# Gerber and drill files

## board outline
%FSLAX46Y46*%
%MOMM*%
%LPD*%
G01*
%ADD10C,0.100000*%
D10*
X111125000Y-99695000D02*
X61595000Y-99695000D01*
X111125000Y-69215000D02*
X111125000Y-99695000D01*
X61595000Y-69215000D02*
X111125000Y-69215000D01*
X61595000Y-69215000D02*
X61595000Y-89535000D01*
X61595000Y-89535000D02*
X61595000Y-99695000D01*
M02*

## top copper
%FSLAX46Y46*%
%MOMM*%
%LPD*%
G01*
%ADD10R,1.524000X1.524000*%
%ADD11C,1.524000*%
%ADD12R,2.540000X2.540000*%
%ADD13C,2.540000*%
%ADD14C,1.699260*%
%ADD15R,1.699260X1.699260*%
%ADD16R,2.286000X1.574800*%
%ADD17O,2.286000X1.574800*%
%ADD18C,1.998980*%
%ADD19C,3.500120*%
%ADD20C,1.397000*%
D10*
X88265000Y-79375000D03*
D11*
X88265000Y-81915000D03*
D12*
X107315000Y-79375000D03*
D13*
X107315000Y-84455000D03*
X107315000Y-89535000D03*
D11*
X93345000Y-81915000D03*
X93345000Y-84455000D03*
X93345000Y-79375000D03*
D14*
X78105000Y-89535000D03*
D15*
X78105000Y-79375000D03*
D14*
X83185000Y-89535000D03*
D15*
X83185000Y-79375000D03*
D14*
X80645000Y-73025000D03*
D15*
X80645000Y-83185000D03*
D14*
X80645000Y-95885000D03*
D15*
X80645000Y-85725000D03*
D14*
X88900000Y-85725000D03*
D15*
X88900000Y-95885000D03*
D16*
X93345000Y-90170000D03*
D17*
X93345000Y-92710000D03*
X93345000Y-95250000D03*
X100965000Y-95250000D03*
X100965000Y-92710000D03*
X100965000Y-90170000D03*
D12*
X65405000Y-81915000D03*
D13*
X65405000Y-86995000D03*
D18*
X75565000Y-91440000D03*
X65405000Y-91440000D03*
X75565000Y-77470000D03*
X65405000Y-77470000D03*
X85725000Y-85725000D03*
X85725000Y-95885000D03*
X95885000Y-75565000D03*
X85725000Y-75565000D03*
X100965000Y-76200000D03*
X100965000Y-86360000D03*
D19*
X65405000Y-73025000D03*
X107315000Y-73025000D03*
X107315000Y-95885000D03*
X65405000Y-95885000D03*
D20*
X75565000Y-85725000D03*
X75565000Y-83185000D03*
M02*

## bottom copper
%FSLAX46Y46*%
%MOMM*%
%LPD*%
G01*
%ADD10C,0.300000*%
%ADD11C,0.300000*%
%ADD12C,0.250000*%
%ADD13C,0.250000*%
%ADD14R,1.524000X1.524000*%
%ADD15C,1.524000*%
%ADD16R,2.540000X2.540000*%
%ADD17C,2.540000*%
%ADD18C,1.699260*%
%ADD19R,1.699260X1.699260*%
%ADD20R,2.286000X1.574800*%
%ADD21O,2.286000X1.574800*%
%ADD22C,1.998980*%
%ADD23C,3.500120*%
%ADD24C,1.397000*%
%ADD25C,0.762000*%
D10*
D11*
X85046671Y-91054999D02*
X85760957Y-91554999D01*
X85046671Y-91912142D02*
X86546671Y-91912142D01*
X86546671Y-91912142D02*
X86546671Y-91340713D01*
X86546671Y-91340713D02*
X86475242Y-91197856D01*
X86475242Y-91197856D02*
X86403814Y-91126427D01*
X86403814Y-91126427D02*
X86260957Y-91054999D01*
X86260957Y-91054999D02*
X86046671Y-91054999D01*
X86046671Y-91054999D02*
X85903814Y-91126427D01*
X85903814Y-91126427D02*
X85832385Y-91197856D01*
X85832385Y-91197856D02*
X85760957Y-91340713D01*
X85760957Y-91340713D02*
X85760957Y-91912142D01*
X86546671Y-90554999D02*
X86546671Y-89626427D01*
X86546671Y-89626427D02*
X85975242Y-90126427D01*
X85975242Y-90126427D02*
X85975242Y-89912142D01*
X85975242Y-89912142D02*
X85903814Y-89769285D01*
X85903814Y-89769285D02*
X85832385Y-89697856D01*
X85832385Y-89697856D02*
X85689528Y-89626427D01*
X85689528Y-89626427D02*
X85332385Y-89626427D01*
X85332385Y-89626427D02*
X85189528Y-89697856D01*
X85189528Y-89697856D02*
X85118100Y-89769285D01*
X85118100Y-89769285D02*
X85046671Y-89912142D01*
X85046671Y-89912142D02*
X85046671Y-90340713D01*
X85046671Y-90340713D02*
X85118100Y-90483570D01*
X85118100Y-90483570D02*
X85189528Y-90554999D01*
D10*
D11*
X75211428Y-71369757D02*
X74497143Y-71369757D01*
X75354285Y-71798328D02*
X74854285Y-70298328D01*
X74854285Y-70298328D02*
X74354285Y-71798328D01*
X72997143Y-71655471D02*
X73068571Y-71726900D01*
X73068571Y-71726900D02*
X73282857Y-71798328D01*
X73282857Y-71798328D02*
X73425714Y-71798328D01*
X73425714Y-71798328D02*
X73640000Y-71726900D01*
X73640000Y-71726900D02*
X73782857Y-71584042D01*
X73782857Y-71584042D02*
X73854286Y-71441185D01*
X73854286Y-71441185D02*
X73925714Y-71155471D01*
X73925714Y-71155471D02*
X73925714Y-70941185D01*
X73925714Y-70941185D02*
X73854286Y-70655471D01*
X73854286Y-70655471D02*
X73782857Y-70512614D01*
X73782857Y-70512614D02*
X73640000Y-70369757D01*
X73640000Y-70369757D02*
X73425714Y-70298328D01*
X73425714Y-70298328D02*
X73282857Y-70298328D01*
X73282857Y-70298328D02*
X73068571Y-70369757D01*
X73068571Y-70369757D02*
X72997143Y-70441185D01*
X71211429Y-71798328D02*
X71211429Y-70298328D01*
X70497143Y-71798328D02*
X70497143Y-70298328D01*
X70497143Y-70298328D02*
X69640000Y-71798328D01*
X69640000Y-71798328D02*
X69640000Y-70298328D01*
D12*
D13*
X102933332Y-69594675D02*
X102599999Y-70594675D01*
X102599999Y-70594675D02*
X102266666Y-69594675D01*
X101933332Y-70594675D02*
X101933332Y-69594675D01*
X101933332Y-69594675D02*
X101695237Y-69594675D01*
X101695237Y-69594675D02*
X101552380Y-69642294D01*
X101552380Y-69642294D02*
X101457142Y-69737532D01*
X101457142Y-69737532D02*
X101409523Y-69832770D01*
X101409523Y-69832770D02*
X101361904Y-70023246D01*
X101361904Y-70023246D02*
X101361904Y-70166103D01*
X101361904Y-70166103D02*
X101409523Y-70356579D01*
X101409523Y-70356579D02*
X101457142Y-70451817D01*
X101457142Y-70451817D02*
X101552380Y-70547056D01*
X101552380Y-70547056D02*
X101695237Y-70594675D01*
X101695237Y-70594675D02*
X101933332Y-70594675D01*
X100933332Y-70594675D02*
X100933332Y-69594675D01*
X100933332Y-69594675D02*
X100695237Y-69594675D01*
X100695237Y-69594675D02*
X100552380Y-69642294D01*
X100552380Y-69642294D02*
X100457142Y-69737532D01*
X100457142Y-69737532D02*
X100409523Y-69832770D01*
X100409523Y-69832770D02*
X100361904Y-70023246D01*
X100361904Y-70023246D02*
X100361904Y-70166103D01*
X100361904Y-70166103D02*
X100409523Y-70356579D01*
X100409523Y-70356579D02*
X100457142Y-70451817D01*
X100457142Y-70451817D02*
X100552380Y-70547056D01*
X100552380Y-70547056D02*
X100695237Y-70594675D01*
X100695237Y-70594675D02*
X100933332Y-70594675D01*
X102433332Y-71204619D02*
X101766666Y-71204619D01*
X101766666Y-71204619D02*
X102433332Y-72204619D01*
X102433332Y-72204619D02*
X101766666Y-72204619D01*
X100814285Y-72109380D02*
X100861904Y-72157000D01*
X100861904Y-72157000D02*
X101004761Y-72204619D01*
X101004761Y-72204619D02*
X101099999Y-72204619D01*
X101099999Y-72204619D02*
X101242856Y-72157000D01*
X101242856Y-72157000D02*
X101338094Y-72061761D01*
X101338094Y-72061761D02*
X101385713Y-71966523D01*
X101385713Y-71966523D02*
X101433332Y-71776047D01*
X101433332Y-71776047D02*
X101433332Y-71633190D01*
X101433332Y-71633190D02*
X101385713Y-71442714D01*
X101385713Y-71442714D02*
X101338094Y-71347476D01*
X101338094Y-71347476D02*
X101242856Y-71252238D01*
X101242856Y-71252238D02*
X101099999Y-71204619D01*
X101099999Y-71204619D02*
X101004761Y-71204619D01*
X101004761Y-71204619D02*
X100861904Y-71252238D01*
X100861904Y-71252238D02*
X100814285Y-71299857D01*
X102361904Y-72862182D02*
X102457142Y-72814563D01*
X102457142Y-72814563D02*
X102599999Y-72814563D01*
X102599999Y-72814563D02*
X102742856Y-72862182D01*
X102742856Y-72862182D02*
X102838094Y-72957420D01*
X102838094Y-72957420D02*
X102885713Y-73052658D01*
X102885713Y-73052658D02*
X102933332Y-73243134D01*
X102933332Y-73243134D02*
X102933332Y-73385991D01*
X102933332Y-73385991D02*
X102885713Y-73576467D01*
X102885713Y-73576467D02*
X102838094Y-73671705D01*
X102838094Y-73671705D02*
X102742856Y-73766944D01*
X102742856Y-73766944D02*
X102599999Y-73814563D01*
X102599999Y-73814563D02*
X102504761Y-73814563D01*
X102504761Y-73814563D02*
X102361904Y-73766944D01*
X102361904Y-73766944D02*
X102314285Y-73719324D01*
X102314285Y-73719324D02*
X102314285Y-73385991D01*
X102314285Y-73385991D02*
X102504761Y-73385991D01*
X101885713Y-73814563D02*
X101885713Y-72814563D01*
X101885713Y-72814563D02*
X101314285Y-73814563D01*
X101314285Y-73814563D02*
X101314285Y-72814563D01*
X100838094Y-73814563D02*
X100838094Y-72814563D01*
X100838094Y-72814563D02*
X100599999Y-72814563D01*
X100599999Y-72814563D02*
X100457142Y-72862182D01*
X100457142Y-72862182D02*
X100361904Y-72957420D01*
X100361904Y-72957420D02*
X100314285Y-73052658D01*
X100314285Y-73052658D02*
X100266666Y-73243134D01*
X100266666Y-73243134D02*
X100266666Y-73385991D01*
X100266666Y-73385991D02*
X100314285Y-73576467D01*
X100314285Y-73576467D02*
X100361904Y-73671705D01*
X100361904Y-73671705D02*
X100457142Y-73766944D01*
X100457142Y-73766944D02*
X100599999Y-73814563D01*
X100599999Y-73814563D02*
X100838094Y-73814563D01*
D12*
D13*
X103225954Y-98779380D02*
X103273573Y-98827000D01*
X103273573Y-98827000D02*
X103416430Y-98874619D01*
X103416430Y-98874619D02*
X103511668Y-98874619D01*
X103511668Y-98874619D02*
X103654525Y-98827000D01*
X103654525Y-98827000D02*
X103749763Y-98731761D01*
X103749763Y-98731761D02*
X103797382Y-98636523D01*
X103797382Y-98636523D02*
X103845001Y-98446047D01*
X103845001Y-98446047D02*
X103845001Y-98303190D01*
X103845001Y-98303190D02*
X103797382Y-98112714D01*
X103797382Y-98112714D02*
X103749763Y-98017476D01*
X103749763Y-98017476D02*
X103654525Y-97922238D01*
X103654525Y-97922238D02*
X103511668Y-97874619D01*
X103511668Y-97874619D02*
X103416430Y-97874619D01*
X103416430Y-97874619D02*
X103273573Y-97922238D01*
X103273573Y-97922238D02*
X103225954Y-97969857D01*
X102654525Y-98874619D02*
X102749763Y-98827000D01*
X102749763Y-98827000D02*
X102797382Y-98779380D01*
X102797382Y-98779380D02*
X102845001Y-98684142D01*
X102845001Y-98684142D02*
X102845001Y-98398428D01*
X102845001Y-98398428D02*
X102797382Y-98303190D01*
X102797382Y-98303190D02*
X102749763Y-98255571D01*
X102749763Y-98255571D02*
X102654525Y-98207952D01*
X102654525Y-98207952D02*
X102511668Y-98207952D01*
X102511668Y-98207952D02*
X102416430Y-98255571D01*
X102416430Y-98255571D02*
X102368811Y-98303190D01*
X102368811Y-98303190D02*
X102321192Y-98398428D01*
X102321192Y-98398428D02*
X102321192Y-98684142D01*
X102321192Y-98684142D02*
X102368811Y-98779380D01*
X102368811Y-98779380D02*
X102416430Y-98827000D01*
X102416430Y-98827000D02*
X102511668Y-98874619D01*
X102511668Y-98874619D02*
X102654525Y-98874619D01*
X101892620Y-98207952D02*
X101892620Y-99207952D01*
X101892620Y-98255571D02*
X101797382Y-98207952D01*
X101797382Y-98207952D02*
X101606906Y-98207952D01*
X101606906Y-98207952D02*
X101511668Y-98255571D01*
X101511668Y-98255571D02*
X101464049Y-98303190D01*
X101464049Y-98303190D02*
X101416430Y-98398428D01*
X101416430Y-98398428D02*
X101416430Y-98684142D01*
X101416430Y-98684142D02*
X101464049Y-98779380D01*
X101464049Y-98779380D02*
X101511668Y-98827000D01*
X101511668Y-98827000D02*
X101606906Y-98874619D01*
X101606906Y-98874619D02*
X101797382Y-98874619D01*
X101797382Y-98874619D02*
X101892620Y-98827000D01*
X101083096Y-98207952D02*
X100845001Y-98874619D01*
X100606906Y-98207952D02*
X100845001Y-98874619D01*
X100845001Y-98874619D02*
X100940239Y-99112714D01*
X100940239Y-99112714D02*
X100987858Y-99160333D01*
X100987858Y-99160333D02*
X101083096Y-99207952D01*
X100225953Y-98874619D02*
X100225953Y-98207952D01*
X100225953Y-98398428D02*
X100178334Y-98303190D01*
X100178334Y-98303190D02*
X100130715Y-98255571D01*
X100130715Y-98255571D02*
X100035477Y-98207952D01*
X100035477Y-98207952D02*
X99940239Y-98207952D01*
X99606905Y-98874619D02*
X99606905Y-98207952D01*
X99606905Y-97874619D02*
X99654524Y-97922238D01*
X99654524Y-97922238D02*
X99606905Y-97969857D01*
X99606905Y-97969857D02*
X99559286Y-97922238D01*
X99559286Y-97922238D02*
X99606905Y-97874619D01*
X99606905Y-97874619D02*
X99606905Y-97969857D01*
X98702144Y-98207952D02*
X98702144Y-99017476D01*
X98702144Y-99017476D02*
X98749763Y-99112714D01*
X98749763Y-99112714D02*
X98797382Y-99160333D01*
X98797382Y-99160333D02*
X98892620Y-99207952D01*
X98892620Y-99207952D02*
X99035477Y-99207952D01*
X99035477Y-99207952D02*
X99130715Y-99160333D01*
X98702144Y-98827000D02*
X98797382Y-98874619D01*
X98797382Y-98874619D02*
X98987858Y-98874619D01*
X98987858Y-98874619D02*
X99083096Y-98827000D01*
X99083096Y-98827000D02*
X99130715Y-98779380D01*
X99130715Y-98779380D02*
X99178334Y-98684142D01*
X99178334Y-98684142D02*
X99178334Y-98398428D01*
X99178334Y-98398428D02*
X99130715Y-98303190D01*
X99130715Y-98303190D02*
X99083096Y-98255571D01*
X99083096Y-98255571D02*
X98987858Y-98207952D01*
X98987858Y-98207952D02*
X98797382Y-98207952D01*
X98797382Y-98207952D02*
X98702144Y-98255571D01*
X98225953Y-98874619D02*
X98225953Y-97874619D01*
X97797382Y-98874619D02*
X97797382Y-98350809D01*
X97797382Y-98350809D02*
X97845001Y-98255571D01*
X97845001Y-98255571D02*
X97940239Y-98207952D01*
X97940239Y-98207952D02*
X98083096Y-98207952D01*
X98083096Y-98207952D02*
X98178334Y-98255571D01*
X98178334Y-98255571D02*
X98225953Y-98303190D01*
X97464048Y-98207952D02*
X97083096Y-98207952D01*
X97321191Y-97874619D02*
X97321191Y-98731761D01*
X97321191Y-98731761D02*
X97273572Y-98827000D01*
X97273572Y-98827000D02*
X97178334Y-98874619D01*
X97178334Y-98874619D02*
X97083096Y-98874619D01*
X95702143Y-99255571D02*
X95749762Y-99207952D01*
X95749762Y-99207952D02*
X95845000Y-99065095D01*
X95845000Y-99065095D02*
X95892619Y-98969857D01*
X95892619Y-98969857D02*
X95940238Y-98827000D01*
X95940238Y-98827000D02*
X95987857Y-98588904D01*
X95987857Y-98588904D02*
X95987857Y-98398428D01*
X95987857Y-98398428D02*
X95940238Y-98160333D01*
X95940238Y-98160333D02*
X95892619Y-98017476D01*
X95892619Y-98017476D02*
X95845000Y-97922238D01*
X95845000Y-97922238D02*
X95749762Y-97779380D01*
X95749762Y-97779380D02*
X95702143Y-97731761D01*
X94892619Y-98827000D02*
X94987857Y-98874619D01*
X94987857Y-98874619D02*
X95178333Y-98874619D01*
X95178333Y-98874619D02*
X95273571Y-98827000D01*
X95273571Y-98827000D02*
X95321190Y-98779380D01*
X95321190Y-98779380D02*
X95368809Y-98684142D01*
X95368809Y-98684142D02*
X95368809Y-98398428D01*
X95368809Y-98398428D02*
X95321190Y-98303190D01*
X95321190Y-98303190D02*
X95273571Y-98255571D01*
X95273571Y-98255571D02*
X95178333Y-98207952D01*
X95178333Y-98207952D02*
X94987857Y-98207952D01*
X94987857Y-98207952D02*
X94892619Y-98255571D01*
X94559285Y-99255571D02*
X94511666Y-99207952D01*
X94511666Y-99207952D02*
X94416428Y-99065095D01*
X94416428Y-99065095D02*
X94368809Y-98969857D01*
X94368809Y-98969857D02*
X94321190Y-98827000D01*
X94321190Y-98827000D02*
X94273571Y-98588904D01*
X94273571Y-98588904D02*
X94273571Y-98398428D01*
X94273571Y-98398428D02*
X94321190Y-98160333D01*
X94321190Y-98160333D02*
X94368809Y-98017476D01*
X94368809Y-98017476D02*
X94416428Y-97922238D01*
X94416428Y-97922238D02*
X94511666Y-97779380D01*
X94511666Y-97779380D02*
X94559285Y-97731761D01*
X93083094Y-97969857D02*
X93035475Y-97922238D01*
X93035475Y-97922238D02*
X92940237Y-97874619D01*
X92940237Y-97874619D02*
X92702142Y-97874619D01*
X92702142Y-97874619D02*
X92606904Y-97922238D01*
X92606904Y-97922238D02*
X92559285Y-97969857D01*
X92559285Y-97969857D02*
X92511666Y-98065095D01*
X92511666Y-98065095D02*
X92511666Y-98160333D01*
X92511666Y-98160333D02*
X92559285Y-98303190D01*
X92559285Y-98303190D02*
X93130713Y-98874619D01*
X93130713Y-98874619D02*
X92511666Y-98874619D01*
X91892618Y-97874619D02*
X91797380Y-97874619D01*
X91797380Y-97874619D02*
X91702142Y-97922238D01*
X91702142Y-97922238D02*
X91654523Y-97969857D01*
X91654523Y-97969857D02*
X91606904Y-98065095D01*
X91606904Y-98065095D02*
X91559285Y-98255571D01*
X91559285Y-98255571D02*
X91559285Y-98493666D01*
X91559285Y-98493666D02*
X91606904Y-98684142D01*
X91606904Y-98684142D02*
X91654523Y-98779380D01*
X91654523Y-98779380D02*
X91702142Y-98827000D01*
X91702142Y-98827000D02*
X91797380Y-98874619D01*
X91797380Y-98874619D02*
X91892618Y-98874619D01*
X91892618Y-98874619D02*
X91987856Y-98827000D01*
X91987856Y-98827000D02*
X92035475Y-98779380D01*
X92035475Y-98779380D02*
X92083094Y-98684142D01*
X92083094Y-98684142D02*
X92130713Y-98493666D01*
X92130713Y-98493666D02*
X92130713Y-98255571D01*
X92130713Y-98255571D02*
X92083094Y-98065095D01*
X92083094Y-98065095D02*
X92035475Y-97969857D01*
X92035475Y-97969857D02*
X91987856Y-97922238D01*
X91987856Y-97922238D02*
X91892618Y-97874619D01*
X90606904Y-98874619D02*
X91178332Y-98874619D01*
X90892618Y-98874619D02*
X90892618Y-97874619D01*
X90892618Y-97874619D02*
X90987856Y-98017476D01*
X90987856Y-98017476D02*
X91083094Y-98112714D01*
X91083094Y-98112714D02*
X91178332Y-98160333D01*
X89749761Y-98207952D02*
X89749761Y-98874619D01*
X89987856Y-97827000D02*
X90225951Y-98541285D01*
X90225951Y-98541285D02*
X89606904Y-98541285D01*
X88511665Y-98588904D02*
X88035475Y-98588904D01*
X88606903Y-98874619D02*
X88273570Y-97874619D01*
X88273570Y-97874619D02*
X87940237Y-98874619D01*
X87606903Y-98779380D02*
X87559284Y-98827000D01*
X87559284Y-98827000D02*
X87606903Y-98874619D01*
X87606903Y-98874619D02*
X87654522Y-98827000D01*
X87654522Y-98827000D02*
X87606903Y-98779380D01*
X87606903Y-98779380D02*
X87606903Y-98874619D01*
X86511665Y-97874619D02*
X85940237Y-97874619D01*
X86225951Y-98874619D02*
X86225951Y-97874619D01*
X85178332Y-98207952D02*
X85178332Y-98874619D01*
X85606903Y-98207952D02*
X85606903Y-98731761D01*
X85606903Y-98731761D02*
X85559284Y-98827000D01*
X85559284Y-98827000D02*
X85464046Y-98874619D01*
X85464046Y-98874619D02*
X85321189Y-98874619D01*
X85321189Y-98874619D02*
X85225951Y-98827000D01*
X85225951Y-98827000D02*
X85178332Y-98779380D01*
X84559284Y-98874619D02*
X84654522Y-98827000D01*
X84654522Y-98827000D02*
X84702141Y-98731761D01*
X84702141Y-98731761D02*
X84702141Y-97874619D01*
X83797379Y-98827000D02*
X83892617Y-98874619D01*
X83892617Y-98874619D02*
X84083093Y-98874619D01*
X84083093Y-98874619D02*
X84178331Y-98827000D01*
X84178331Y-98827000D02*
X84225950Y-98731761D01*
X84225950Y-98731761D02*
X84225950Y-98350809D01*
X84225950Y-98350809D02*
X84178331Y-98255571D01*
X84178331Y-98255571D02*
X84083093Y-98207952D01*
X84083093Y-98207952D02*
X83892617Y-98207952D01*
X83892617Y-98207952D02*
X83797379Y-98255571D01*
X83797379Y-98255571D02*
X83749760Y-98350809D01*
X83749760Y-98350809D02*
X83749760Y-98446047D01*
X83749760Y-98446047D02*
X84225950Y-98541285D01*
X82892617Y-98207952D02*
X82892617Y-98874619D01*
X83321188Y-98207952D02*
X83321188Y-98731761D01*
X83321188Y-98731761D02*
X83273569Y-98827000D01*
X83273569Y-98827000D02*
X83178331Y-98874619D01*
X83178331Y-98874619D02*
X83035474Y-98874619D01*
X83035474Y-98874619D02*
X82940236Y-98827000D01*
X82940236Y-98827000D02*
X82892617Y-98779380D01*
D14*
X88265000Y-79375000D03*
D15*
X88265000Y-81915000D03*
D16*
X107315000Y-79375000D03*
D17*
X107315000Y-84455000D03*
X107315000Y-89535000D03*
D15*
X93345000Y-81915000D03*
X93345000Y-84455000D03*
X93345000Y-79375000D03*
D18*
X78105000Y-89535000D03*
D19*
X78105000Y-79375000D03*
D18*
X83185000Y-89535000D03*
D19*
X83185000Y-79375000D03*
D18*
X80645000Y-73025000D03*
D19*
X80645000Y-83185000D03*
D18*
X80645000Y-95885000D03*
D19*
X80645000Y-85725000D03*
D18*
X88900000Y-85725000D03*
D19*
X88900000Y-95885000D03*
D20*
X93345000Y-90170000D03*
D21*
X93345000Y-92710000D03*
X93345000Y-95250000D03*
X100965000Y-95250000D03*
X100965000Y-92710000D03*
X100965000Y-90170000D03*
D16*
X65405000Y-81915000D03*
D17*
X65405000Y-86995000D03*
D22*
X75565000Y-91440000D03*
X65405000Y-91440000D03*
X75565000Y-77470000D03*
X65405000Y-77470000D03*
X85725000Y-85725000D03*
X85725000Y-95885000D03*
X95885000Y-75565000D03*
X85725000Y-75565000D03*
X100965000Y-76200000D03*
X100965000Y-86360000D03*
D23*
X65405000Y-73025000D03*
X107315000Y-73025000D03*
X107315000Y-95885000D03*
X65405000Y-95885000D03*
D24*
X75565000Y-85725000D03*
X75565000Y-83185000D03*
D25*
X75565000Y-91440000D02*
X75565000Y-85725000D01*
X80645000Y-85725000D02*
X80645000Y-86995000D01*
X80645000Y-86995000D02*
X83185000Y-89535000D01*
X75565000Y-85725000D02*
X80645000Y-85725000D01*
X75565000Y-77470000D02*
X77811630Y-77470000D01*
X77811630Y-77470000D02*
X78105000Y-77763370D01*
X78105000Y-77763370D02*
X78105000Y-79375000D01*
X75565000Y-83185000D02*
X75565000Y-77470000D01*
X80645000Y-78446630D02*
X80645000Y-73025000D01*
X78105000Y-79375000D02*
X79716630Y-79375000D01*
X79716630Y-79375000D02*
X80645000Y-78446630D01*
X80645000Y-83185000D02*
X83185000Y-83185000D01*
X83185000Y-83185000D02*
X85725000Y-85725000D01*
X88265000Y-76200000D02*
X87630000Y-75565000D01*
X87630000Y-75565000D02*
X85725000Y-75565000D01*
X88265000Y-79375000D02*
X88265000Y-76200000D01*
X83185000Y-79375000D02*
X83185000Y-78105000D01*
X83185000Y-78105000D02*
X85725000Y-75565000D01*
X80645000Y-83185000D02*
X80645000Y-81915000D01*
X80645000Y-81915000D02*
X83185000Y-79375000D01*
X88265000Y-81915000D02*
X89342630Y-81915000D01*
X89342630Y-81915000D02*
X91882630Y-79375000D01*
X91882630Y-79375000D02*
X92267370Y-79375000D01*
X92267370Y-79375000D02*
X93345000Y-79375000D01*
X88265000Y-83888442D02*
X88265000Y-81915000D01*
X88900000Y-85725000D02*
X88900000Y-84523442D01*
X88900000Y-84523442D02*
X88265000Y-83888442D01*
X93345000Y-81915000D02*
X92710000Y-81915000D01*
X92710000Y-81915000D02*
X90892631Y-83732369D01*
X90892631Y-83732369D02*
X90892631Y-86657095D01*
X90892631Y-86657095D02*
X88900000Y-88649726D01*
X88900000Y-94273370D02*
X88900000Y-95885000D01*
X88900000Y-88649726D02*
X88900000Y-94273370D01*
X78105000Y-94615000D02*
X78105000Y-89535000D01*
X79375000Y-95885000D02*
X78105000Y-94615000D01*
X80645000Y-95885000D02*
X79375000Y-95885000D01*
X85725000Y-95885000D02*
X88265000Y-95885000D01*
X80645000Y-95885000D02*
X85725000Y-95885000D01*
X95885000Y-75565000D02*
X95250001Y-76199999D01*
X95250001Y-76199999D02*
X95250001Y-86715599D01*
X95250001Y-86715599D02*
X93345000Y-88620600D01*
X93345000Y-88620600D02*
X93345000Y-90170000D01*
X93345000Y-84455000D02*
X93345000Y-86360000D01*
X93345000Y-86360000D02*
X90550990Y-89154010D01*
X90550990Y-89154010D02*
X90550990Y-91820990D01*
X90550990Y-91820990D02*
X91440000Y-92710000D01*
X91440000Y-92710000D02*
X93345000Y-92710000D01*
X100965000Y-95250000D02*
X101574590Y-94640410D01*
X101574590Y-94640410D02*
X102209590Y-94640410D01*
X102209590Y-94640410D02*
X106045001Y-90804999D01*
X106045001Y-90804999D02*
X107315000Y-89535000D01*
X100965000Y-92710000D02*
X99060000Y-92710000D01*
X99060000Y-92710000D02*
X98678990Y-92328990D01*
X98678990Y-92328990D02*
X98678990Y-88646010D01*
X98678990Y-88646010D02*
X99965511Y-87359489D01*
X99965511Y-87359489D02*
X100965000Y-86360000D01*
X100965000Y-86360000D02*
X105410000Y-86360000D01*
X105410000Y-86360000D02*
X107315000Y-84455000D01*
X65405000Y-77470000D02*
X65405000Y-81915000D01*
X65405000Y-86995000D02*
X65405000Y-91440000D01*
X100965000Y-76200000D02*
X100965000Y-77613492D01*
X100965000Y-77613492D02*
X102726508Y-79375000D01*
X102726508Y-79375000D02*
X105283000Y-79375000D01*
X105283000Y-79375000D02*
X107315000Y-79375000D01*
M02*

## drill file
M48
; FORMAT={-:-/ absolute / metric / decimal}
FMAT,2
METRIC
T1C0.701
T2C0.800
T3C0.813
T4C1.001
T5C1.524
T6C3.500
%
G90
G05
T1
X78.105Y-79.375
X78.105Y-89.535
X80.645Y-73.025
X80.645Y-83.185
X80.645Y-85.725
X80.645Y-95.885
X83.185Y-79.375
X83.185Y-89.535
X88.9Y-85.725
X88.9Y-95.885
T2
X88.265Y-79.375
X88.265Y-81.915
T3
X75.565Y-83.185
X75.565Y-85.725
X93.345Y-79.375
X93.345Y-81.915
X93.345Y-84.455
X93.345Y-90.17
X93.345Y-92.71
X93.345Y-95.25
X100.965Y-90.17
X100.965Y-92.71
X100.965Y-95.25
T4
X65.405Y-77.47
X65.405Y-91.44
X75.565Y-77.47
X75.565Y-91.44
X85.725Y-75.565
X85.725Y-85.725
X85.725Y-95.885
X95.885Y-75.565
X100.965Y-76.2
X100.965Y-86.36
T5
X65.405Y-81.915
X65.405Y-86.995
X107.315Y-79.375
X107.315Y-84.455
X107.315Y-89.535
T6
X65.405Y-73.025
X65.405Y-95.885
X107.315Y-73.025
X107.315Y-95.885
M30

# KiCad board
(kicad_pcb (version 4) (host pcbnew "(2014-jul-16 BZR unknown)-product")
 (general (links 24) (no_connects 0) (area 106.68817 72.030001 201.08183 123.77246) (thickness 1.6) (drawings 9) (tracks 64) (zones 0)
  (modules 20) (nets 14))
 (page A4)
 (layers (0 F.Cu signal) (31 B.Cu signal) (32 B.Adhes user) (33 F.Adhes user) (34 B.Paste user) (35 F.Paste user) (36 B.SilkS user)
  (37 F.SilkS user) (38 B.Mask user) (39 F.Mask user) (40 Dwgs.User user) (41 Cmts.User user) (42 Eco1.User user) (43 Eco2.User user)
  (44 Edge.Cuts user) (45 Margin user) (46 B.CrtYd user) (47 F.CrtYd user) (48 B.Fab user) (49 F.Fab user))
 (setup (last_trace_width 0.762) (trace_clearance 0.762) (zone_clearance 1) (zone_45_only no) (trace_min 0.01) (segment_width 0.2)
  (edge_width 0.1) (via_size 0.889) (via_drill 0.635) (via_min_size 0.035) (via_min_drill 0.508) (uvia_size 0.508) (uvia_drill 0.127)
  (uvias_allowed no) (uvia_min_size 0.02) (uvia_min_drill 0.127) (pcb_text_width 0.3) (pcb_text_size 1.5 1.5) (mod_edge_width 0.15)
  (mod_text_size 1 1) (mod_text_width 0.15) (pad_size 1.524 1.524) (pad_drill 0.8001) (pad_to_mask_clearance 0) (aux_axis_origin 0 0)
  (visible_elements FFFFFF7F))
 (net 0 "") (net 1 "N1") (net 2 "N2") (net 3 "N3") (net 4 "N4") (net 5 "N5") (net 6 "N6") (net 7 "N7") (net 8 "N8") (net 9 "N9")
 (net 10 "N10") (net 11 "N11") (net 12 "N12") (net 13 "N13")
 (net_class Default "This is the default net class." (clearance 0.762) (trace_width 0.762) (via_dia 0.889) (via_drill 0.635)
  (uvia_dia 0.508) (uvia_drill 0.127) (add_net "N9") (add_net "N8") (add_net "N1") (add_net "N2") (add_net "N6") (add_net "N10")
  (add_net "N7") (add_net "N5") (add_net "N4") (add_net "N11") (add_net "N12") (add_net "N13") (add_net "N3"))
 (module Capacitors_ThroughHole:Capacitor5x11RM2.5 (layer F.Cu) (at 88.265 80.645 180)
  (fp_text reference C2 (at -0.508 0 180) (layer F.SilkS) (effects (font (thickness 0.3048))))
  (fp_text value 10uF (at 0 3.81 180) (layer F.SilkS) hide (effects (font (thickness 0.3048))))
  (pad 1 thru_hole rect (at 0 1.27 180) (size 1.524 1.524) (drill 0.8001) (layers *.Cu *.Mask F.SilkS) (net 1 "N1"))
  (pad 2 thru_hole circle (at 0 -1.27 180) (size 1.524 1.524) (drill 0.8001) (layers *.Cu *.Mask F.SilkS) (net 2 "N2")))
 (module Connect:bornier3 (layer F.Cu) (at 107.315 84.455 270)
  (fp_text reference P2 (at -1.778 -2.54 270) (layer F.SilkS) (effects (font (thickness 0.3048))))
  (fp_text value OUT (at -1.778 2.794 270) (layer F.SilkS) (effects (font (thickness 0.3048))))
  (pad 1 thru_hole rect (at -5.08 0 270) (size 2.54 2.54) (drill 1.524) (layers *.Cu *.Mask F.SilkS) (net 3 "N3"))
  (pad 2 thru_hole circle (at 0 0 270) (size 2.54 2.54) (drill 1.524) (layers *.Cu *.Mask F.SilkS) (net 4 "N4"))
  (pad 3 thru_hole circle (at 5.08 0 270) (size 2.54 2.54) (drill 1.524) (layers *.Cu *.Mask F.SilkS) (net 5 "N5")))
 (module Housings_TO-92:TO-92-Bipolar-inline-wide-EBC (layer F.Cu) (at 93.345 81.915)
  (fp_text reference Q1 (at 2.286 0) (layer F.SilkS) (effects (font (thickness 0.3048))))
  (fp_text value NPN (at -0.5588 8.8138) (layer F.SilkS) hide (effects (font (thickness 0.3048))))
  (pad B thru_hole circle (at 0 0) (size 1.524 1.524) (drill 0.8128) (layers *.Cu *.Mask F.SilkS) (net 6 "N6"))
  (pad C thru_hole circle (at 0 2.54) (size 1.524 1.524) (drill 0.8128) (layers *.Cu *.Mask F.SilkS) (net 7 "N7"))
  (pad E thru_hole circle (at 0 -2.54) (size 1.524 1.524) (drill 0.8128) (layers *.Cu *.Mask F.SilkS) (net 2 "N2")))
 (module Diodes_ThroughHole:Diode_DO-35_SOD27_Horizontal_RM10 (layer F.Cu) (at 78.105 84.455 90)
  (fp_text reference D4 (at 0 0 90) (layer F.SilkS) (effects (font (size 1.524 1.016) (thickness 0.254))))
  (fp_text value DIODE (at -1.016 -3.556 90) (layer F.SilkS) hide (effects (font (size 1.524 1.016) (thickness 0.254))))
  (pad 1 thru_hole circle (at -5.08 0 90) (size 1.69926 1.69926) (drill 0.70104) (layers *.Cu *.Mask F.SilkS) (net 6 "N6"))
  (pad 2 thru_hole rect (at 5.08 0 90) (size 1.69926 1.69926) (drill 0.70104) (layers *.Cu *.Mask F.SilkS) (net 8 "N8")))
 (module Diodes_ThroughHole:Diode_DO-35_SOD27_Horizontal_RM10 (layer F.Cu) (at 83.185 84.455 90)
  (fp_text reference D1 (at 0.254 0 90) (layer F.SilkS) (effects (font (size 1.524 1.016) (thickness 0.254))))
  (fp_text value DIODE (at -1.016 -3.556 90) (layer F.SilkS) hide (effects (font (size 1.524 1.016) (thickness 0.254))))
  (pad 1 thru_hole circle (at -5.08 0 90) (size 1.69926 1.69926) (drill 0.70104) (layers *.Cu *.Mask F.SilkS) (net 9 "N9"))
  (pad 2 thru_hole rect (at 5.08 0 90) (size 1.69926 1.69926) (drill 0.70104) (layers *.Cu *.Mask F.SilkS) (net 1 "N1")))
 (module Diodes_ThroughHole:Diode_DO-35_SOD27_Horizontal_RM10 (layer F.Cu) (at 80.645 78.105 270)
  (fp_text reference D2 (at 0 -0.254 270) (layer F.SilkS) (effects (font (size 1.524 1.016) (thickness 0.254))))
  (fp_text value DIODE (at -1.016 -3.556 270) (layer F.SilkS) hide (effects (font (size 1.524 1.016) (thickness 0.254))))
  (pad 1 thru_hole circle (at -5.08 0 270) (size 1.69926 1.69926) (drill 0.70104) (layers *.Cu *.Mask F.SilkS) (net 8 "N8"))
  (pad 2 thru_hole rect (at 5.08 0 270) (size 1.69926 1.69926) (drill 0.70104) (layers *.Cu *.Mask F.SilkS) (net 1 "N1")))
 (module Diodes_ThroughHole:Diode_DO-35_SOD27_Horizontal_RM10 (layer F.Cu) (at 80.645 90.805 90)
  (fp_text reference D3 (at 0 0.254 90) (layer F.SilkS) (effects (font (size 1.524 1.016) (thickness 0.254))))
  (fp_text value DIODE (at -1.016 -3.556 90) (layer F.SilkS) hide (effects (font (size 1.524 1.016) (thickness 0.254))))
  (pad 1 thru_hole circle (at -5.08 0 90) (size 1.69926 1.69926) (drill 0.70104) (layers *.Cu *.Mask F.SilkS) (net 6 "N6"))
  (pad 2 thru_hole rect (at 5.08 0 90) (size 1.69926 1.69926) (drill 0.70104) (layers *.Cu *.Mask F.SilkS) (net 9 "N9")))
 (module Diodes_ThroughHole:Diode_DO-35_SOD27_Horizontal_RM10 (layer F.Cu) (at 88.9 90.805 270)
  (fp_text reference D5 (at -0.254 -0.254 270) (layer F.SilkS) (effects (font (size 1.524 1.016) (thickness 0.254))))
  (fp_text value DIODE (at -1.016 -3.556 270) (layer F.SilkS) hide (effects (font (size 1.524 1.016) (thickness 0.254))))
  (pad 1 thru_hole circle (at -5.08 0 270) (size 1.69926 1.69926) (drill 0.70104) (layers *.Cu *.Mask F.SilkS) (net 2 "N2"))
  (pad 2 thru_hole rect (at 5.08 0 270) (size 1.69926 1.69926) (drill 0.70104) (layers *.Cu *.Mask F.SilkS) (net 6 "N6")))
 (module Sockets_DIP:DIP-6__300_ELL (layer F.Cu) (at 97.155 92.71 270)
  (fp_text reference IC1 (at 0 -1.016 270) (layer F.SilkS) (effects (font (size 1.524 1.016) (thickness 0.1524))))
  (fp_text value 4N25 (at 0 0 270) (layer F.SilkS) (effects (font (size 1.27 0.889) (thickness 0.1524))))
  (pad 1 thru_hole rect (at -2.54 3.81 270) (size 1.5748 2.286) (drill 0.8128) (layers *.Cu *.Mask F.SilkS) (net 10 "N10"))
  (pad 2 thru_hole oval (at 0 3.81 270) (size 1.5748 2.286) (drill 0.8128) (layers *.Cu *.Mask F.SilkS) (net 7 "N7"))
  (pad 3 thru_hole oval (at 2.54 3.81 270) (size 1.5748 2.286) (drill 0.8128) (layers *.Cu *.Mask F.SilkS))
  (pad 4 thru_hole oval (at 2.54 -3.81 270) (size 1.5748 2.286) (drill 0.8128) (layers *.Cu *.Mask F.SilkS) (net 5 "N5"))
  (pad 5 thru_hole oval (at 0 -3.81 270) (size 1.5748 2.286) (drill 0.8128) (layers *.Cu *.Mask F.SilkS) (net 4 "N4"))
  (pad 6 thru_hole oval (at -2.54 -3.81 270) (size 1.5748 2.286) (drill 0.8128) (layers *.Cu *.Mask F.SilkS) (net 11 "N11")))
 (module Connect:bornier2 (layer F.Cu) (at 65.405 84.455 270)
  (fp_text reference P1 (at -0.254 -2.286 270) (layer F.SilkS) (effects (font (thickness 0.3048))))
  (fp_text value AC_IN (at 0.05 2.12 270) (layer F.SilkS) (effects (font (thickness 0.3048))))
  (pad 1 thru_hole rect (at -2.54 0 270) (size 2.54 2.54) (drill 1.524) (layers *.Cu *.Mask F.SilkS) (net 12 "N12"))
  (pad 2 thru_hole circle (at 2.54 0 270) (size 2.54 2.54) (drill 1.524) (layers *.Cu *.Mask F.SilkS) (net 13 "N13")))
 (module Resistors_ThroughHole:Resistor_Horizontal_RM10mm (layer F.Cu) (at 70.485 91.44 180)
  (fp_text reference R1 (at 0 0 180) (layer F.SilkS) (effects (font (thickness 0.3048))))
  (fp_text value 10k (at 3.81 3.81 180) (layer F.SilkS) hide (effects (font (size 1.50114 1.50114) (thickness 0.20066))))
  (pad 1 thru_hole circle (at -5.08 0 180) (size 1.99898 1.99898) (drill 1.00076) (layers *.Cu *.SilkS *.Mask) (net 9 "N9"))
  (pad 2 thru_hole circle (at 5.08 0 180) (size 1.99898 1.99898) (drill 1.00076) (layers *.Cu *.SilkS *.Mask) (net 13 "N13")))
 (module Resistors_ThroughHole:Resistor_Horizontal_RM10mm (layer F.Cu) (at 70.485 77.47 180)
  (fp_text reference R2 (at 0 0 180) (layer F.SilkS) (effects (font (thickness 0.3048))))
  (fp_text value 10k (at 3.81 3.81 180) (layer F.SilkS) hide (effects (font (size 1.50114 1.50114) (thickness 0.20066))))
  (pad 1 thru_hole circle (at -5.08 0 180) (size 1.99898 1.99898) (drill 1.00076) (layers *.Cu *.SilkS *.Mask) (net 8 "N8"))
  (pad 2 thru_hole circle (at 5.08 0 180) (size 1.99898 1.99898) (drill 1.00076) (layers *.Cu *.SilkS *.Mask) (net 12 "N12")))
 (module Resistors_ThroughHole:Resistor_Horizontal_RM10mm (layer F.Cu) (at 85.725 90.805 270)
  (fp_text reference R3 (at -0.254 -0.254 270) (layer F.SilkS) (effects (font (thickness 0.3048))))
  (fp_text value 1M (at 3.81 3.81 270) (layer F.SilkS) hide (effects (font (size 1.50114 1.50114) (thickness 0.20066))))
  (pad 1 thru_hole circle (at -5.08 0 270) (size 1.99898 1.99898) (drill 1.00076) (layers *.Cu *.SilkS *.Mask) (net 1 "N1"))
  (pad 2 thru_hole circle (at 5.08 0 270) (size 1.99898 1.99898) (drill 1.00076) (layers *.Cu *.SilkS *.Mask) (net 6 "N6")))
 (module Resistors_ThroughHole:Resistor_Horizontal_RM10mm (layer F.Cu) (at 90.805 75.565 180)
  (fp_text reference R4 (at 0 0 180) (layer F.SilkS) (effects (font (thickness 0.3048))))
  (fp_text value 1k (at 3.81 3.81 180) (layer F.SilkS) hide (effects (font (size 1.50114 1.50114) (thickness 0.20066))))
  (pad 1 thru_hole circle (at -5.08 0 180) (size 1.99898 1.99898) (drill 1.00076) (layers *.Cu *.SilkS *.Mask) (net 10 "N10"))
  (pad 2 thru_hole circle (at 5.08 0 180) (size 1.99898 1.99898) (drill 1.00076) (layers *.Cu *.SilkS *.Mask) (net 1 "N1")))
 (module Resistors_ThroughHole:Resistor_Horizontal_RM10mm (layer F.Cu) (at 100.965 81.28 270)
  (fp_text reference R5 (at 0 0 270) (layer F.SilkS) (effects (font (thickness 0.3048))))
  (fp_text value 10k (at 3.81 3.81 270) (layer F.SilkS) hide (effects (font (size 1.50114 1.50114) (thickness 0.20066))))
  (pad 1 thru_hole circle (at -5.08 0 270) (size 1.99898 1.99898) (drill 1.00076) (layers *.Cu *.SilkS *.Mask) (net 3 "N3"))
  (pad 2 thru_hole circle (at 5.08 0 270) (size 1.99898 1.99898) (drill 1.00076) (layers *.Cu *.SilkS *.Mask) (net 4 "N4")))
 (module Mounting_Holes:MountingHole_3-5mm (layer F.Cu) (at 65.405 73.025)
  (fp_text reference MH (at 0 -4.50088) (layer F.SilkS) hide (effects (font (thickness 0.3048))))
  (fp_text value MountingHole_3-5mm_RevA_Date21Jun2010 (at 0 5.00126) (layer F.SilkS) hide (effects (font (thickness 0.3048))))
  (pad 1 thru_hole circle (at 0 0) (size 3.50012 3.50012) (drill 3.50012) (layers)))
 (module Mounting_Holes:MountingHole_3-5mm (layer F.Cu) (at 107.315 73.025)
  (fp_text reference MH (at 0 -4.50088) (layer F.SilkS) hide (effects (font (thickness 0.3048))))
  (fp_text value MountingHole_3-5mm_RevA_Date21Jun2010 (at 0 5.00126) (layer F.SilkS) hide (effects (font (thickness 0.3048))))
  (pad 1 thru_hole circle (at 0 0) (size 3.50012 3.50012) (drill 3.50012) (layers)))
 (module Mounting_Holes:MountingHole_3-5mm (layer F.Cu) (at 107.315 95.885)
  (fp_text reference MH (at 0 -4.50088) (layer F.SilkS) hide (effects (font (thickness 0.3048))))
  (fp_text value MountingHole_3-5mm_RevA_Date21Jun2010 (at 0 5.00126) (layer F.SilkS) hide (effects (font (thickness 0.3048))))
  (pad 1 thru_hole circle (at 0 0) (size 3.50012 3.50012) (drill 3.50012) (layers)))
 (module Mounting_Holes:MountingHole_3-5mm (layer F.Cu) (at 65.405 95.885)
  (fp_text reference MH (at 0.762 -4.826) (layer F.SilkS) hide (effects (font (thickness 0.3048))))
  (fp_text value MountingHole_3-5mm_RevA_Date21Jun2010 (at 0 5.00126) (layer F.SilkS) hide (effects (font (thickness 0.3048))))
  (pad 1 thru_hole circle (at 0 0) (size 3.50012 3.50012) (drill 3.50012) (layers)))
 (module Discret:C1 (layer F.Cu) (at 75.565 84.455 90)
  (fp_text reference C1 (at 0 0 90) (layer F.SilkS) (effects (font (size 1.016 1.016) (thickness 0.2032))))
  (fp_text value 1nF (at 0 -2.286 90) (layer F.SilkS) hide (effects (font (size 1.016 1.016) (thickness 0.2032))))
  (pad 1 thru_hole circle (at -1.27 0 90) (size 1.397 1.397) (drill 0.8128) (layers *.Cu *.Mask F.SilkS) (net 9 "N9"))
  (pad 2 thru_hole circle (at 1.27 0 90) (size 1.397 1.397) (drill 0.8128) (layers *.Cu *.Mask F.SilkS) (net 8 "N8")))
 (gr_line (start 111.125 99.695) (end 61.595 99.695) (layer Edge.Cuts) (width 0.1))
 (gr_line (start 111.125 69.215) (end 111.125 99.695) (layer Edge.Cuts) (width 0.1))
 (gr_line (start 61.595 69.215) (end 111.125 69.215) (layer Edge.Cuts) (width 0.1))
 (gr_line (start 61.595 69.215) (end 61.595 89.535) (layer Edge.Cuts) (width 0.1))
 (gr_line (start 61.595 89.535) (end 61.595 99.695) (layer Edge.Cuts) (width 0.1))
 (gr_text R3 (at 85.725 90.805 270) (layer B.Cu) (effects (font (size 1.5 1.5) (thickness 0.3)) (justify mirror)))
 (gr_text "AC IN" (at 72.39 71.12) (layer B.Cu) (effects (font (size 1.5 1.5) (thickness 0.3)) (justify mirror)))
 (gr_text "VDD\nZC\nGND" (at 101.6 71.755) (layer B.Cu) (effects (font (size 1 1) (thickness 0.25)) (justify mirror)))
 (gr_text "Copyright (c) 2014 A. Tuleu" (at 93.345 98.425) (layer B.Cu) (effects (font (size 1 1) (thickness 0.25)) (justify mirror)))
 (segment (start 75.565 91.44) (end 75.565 85.725) (width 0.762) (layer B.Cu) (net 9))
 (segment (start 80.645 85.725) (end 80.645 86.995) (width 0.762) (layer B.Cu) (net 9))
 (segment (start 80.645 86.995) (end 83.185 89.535) (width 0.762) (layer B.Cu) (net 9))
 (segment (start 75.565 85.725) (end 80.645 85.725) (width 0.762) (layer B.Cu) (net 9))
 (segment (start 75.565 77.47) (end 77.81163 77.47) (width 0.762) (layer B.Cu) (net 8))
 (segment (start 77.81163 77.47) (end 78.105 77.76337) (width 0.762) (layer B.Cu) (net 8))
 (segment (start 78.105 77.76337) (end 78.105 79.375) (width 0.762) (layer B.Cu) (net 8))
 (segment (start 75.565 83.185) (end 75.565 77.47) (width 0.762) (layer B.Cu) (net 8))
 (segment (start 80.645 78.44663) (end 80.645 73.025) (width 0.762) (layer B.Cu) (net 8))
 (segment (start 78.105 79.375) (end 79.71663 79.375) (width 0.762) (layer B.Cu) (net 8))
 (segment (start 79.71663 79.375) (end 80.645 78.44663) (width 0.762) (layer B.Cu) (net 8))
 (segment (start 80.645 83.185) (end 83.185 83.185) (width 0.762) (layer B.Cu) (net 1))
 (segment (start 83.185 83.185) (end 85.725 85.725) (width 0.762) (layer B.Cu) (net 1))
 (segment (start 88.265 76.2) (end 87.63 75.565) (width 0.762) (layer B.Cu) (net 1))
 (segment (start 87.63 75.565) (end 85.725 75.565) (width 0.762) (layer B.Cu) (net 1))
 (segment (start 88.265 79.375) (end 88.265 76.2) (width 0.762) (layer B.Cu) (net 1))
 (segment (start 83.185 79.375) (end 83.185 78.105) (width 0.762) (layer B.Cu) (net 1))
 (segment (start 83.185 78.105) (end 85.725 75.565) (width 0.762) (layer B.Cu) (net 1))
 (segment (start 80.645 83.185) (end 80.645 81.915) (width 0.762) (layer B.Cu) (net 1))
 (segment (start 80.645 81.915) (end 83.185 79.375) (width 0.762) (layer B.Cu) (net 1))
 (segment (start 88.265 81.915) (end 89.34263 81.915) (width 0.762) (layer B.Cu) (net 2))
 (segment (start 89.34263 81.915) (end 91.88263 79.375) (width 0.762) (layer B.Cu) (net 2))
 (segment (start 91.88263 79.375) (end 92.26737 79.375) (width 0.762) (layer B.Cu) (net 2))
 (segment (start 92.26737 79.375) (end 93.345 79.375) (width 0.762) (layer B.Cu) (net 2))
 (segment (start 88.265 83.888442) (end 88.265 81.915) (width 0.762) (layer B.Cu) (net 2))
 (segment (start 88.9 85.725) (end 88.9 84.523442) (width 0.762) (layer B.Cu) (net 2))
 (segment (start 88.9 84.523442) (end 88.265 83.888442) (width 0.762) (layer B.Cu) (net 2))
 (segment (start 93.345 81.915) (end 92.71 81.915) (width 0.762) (layer B.Cu) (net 6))
 (segment (start 92.71 81.915) (end 90.892631 83.732369) (width 0.762) (layer B.Cu) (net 6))
 (segment (start 90.892631 83.732369) (end 90.892631 86.657095) (width 0.762) (layer B.Cu) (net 6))
 (segment (start 90.892631 86.657095) (end 88.9 88.649726) (width 0.762) (layer B.Cu) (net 6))
 (segment (start 88.9 94.27337) (end 88.9 95.885) (width 0.762) (layer B.Cu) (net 6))
 (segment (start 88.9 88.649726) (end 88.9 94.27337) (width 0.762) (layer B.Cu) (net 6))
 (segment (start 78.105 94.615) (end 78.105 89.535) (width 0.762) (layer B.Cu) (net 6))
 (segment (start 79.375 95.885) (end 78.105 94.615) (width 0.762) (layer B.Cu) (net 6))
 (segment (start 80.645 95.885) (end 79.375 95.885) (width 0.762) (layer B.Cu) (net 6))
 (segment (start 85.725 95.885) (end 88.265 95.885) (width 0.762) (layer B.Cu) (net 6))
 (segment (start 80.645 95.885) (end 85.725 95.885) (width 0.762) (layer B.Cu) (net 6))
 (segment (start 95.885 75.565) (end 95.250001 76.199999) (width 0.762) (layer B.Cu) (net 10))
 (segment (start 95.250001 76.199999) (end 95.250001 86.715599) (width 0.762) (layer B.Cu) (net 10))
 (segment (start 95.250001 86.715599) (end 93.345 88.6206) (width 0.762) (layer B.Cu) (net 10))
 (segment (start 93.345 88.6206) (end 93.345 90.17) (width 0.762) (layer B.Cu) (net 10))
 (segment (start 93.345 84.455) (end 93.345 86.36) (width 0.762) (layer B.Cu) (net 7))
 (segment (start 93.345 86.36) (end 90.55099 89.15401) (width 0.762) (layer B.Cu) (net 7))
 (segment (start 90.55099 89.15401) (end 90.55099 91.82099) (width 0.762) (layer B.Cu) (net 7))
 (segment (start 90.55099 91.82099) (end 91.44 92.71) (width 0.762) (layer B.Cu) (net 7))
 (segment (start 91.44 92.71) (end 93.345 92.71) (width 0.762) (layer B.Cu) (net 7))
 (segment (start 100.965 95.25) (end 101.57459 94.64041) (width 0.762) (layer B.Cu) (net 5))
 (segment (start 101.57459 94.64041) (end 102.20959 94.64041) (width 0.762) (layer B.Cu) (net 5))
 (segment (start 102.20959 94.64041) (end 106.045001 90.804999) (width 0.762) (layer B.Cu) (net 5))
 (segment (start 106.045001 90.804999) (end 107.315 89.535) (width 0.762) (layer B.Cu) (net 5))
 (segment (start 100.965 92.71) (end 99.06 92.71) (width 0.762) (layer B.Cu) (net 4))
 (segment (start 99.06 92.71) (end 98.67899 92.32899) (width 0.762) (layer B.Cu) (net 4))
 (segment (start 98.67899 92.32899) (end 98.67899 88.64601) (width 0.762) (layer B.Cu) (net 4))
 (segment (start 98.67899 88.64601) (end 99.965511 87.359489) (width 0.762) (layer B.Cu) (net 4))
 (segment (start 99.965511 87.359489) (end 100.965 86.36) (width 0.762) (layer B.Cu) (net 4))
 (segment (start 100.965 86.36) (end 105.41 86.36) (width 0.762) (layer B.Cu) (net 4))
 (segment (start 105.41 86.36) (end 107.315 84.455) (width 0.762) (layer B.Cu) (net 4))
 (segment (start 65.405 77.47) (end 65.405 81.915) (width 0.762) (layer B.Cu) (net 12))
 (segment (start 65.405 86.995) (end 65.405 91.44) (width 0.762) (layer B.Cu) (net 13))
 (segment (start 100.965 76.2) (end 100.965 77.613492) (width 0.762) (layer B.Cu) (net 3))
 (segment (start 100.965 77.613492) (end 102.726508 79.375) (width 0.762) (layer B.Cu) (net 3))
 (segment (start 102.726508 79.375) (end 105.283 79.375) (width 0.762) (layer B.Cu) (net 3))
 (segment (start 105.283 79.375) (end 107.315 79.375) (width 0.762) (layer B.Cu) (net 3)))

